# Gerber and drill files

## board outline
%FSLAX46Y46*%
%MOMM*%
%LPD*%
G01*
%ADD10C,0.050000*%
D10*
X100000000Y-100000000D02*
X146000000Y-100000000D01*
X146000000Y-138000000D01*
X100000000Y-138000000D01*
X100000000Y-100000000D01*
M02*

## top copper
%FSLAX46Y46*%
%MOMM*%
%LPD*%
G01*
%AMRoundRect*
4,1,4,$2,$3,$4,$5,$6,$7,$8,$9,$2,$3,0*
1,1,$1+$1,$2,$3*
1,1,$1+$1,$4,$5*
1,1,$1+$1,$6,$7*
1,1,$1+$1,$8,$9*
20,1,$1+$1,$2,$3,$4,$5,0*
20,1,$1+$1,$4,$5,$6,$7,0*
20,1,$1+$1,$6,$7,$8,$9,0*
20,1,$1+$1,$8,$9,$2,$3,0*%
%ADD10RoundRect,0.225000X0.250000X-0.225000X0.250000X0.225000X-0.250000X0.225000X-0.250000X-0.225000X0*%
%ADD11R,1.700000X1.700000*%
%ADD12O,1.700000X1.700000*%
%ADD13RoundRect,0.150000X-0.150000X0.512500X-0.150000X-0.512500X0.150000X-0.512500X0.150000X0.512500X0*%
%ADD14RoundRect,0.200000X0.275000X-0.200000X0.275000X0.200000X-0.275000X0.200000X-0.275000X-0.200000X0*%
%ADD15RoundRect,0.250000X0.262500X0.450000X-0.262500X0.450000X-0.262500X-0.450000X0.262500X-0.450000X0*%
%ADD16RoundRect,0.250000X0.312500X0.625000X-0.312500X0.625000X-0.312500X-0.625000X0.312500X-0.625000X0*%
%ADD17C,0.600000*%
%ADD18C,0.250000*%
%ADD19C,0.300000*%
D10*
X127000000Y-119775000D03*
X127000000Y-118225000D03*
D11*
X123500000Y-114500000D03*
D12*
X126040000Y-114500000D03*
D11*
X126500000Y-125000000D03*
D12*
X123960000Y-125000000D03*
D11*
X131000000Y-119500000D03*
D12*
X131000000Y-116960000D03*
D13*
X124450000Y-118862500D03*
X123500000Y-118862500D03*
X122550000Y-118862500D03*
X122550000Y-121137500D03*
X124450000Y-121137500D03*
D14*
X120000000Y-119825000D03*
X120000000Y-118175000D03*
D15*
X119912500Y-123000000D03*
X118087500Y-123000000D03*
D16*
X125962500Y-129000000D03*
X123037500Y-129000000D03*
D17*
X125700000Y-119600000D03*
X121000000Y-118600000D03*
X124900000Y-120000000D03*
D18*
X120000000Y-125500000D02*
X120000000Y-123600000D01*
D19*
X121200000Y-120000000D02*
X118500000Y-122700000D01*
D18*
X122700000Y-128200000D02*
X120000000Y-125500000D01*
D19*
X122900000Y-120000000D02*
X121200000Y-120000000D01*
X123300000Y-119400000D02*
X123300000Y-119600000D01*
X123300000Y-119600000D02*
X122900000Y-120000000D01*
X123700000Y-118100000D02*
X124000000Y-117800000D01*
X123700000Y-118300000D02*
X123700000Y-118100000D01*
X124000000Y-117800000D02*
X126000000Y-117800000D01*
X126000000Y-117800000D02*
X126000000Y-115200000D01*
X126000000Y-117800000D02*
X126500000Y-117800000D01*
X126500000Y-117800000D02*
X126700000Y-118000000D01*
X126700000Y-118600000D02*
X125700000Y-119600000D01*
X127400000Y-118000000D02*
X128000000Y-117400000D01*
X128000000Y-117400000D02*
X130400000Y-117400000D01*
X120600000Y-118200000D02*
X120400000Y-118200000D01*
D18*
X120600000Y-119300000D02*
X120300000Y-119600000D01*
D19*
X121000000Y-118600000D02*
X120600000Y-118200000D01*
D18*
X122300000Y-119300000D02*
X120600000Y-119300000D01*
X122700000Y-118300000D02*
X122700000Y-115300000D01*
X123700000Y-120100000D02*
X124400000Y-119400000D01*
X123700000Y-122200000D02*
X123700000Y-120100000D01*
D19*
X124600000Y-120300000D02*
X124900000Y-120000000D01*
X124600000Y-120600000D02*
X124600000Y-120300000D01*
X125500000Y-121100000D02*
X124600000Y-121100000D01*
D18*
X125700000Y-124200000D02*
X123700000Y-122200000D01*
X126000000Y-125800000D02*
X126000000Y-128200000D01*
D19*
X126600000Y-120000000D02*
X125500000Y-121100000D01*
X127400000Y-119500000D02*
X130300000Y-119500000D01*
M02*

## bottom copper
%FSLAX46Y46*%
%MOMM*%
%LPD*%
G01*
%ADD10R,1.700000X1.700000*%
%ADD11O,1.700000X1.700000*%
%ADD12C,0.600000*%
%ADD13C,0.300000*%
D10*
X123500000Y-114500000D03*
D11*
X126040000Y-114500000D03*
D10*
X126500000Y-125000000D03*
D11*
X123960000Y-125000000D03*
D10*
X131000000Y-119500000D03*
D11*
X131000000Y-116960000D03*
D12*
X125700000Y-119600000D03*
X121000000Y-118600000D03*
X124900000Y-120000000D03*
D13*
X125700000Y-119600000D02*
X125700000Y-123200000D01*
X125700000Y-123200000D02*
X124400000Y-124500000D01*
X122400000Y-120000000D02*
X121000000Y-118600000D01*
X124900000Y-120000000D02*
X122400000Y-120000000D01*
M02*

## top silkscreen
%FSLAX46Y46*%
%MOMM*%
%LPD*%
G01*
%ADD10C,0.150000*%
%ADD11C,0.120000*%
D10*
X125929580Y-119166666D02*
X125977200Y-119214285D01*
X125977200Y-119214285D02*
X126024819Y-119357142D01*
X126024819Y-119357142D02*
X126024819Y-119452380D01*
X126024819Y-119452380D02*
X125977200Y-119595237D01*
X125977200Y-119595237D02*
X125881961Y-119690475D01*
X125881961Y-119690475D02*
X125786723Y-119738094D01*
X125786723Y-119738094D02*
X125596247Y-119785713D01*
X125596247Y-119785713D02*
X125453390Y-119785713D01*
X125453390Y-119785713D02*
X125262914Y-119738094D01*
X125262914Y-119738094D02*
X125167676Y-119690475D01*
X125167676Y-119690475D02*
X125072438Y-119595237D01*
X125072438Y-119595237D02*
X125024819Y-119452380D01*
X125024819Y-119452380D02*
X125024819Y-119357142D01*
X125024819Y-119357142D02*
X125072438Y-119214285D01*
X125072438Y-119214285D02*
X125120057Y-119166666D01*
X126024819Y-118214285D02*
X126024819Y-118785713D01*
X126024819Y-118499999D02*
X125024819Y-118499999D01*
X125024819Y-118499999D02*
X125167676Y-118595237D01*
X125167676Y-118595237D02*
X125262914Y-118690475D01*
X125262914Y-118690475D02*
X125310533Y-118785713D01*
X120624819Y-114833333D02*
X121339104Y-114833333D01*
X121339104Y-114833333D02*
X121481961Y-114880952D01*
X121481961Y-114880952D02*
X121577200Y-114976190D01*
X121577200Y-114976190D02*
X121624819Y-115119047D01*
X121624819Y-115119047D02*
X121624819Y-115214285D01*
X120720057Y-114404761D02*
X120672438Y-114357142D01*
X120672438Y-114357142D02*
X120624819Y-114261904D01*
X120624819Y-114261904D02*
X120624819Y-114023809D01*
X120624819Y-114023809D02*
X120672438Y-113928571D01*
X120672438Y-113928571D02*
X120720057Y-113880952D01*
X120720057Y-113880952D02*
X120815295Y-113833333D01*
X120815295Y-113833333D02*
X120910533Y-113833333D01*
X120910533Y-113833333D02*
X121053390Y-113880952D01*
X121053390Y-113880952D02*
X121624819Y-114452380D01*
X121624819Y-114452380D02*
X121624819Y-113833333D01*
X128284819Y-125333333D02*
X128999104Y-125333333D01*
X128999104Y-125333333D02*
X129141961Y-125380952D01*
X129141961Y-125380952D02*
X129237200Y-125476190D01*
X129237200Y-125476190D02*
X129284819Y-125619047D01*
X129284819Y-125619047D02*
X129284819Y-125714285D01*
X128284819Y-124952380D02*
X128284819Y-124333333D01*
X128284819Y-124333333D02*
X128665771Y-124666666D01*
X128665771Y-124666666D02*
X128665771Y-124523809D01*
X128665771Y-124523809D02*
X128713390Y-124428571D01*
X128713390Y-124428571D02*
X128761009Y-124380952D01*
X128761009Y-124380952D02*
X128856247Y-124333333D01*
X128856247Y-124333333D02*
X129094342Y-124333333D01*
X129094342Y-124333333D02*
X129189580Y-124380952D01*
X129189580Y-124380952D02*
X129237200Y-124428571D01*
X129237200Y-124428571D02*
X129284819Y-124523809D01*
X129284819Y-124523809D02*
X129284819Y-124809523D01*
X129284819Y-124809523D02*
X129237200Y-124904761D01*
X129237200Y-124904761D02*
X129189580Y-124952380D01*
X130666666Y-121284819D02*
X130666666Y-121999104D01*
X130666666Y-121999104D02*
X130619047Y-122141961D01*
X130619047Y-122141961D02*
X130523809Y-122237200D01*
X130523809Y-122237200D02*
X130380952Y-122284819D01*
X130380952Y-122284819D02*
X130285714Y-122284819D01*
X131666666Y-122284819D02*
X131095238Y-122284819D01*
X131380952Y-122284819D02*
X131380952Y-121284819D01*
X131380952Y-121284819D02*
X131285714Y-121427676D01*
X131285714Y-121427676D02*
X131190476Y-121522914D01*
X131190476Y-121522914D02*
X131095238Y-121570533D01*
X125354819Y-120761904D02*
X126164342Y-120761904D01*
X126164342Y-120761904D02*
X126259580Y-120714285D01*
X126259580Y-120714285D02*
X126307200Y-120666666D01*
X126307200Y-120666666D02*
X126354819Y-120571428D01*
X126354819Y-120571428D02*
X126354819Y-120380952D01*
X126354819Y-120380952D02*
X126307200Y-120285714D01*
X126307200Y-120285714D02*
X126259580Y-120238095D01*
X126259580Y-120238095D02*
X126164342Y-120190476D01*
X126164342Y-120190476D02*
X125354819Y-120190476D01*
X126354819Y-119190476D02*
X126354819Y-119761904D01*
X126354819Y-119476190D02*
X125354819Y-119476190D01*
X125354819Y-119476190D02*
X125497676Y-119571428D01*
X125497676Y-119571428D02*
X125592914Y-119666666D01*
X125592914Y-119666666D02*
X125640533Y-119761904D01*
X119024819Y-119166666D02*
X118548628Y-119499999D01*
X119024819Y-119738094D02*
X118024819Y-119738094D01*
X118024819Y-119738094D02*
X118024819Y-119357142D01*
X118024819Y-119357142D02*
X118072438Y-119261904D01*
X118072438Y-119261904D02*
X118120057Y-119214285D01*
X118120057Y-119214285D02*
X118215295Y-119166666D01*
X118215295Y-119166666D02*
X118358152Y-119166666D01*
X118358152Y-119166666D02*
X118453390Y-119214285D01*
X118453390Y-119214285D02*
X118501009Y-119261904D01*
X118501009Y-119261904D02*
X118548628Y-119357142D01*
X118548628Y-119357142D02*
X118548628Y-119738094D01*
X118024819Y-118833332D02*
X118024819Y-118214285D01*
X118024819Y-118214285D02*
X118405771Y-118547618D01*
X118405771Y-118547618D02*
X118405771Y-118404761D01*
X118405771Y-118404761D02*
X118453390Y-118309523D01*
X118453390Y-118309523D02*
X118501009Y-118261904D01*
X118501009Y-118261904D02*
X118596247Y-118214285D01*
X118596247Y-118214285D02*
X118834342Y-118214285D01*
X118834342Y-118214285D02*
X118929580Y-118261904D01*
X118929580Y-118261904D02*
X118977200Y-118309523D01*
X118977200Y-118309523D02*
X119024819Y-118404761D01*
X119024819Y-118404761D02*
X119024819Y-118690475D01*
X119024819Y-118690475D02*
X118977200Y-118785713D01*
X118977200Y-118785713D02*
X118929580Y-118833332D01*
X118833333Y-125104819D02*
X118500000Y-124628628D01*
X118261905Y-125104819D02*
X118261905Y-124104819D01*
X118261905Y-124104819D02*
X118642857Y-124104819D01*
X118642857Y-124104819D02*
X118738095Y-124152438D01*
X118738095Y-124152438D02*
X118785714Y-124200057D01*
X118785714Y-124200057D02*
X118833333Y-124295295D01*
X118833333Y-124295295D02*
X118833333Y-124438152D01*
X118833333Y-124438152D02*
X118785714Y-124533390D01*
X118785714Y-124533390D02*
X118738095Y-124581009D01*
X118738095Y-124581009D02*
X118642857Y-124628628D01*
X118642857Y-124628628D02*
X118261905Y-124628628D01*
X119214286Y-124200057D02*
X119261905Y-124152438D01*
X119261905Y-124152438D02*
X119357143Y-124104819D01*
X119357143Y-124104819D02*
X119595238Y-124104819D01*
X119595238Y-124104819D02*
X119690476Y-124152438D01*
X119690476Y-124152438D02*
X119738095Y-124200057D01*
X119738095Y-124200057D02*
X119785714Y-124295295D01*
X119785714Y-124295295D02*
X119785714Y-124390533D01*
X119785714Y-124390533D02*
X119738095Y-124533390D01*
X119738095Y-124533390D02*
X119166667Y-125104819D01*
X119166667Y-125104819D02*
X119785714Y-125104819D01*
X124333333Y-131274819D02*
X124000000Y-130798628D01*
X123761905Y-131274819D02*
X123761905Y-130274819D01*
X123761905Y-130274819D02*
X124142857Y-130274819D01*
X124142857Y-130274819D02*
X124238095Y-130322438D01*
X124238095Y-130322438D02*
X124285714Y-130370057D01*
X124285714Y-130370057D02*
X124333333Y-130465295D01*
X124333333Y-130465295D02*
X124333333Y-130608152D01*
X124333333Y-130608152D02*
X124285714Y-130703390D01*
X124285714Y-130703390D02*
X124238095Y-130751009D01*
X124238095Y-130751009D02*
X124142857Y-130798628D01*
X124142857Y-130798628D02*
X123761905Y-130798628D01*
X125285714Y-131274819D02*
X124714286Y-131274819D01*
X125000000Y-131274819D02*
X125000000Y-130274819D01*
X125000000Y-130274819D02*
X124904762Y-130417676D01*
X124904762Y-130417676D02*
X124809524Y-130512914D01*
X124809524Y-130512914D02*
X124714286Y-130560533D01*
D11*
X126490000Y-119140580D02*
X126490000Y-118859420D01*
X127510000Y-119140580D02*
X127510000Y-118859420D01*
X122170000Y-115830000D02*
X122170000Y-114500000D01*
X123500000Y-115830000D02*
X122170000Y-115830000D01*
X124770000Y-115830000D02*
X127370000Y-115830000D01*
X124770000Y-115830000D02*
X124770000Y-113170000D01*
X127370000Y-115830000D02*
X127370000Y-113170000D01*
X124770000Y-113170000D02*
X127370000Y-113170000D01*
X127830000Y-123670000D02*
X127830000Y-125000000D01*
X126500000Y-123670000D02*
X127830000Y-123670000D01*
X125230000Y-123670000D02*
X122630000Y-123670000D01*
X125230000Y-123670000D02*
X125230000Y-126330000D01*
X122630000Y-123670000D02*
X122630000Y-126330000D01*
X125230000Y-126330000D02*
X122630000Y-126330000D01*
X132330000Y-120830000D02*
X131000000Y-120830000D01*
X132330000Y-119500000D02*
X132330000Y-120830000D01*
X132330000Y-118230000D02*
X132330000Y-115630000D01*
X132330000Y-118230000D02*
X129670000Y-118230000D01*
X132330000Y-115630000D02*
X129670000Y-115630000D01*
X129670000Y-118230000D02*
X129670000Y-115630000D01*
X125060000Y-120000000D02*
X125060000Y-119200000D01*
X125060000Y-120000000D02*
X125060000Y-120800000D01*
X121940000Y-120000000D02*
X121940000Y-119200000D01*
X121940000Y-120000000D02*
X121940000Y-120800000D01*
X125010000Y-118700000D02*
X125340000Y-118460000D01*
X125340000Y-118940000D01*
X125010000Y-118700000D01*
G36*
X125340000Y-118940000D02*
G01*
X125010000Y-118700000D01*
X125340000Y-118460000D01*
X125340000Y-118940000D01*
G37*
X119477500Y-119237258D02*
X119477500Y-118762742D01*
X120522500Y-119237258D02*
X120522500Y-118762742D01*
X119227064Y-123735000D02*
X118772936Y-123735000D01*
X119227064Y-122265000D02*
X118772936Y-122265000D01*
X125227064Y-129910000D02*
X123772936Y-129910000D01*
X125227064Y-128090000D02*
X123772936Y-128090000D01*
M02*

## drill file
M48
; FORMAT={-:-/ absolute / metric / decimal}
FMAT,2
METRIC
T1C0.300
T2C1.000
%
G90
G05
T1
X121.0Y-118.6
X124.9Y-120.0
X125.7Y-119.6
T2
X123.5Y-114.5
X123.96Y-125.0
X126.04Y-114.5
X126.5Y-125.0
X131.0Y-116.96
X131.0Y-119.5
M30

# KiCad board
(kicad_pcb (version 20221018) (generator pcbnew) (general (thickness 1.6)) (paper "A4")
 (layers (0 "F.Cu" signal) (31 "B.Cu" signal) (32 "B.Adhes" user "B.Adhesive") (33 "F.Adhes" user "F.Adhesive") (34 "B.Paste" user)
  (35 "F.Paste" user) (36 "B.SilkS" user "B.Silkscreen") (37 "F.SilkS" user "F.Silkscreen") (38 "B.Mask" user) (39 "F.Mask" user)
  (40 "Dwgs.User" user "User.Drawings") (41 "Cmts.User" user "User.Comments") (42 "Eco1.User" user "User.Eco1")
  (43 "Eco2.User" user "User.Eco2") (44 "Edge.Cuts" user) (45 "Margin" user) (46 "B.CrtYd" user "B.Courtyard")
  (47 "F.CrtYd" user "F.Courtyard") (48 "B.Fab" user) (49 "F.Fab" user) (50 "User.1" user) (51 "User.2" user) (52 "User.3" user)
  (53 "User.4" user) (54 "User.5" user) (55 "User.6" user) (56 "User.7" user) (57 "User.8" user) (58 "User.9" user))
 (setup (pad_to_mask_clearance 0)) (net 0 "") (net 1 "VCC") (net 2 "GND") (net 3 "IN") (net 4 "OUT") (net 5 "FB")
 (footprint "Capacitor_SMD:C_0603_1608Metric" (layer "F.Cu") (at 127 119 90)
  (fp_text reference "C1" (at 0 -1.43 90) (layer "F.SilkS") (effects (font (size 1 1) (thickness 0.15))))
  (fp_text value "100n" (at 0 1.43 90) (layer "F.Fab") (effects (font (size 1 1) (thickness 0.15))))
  (fp_line (start -0.14058 -0.51) (end 0.14058 -0.51) (stroke (width 0.12) (type solid)) (layer "F.SilkS"))
  (fp_line (start -0.14058 0.51) (end 0.14058 0.51) (stroke (width 0.12) (type solid)) (layer "F.SilkS"))
  (pad "1" smd roundrect (at -0.775 0 90) (size 0.9 0.95) (layers "F.Cu" "F.Paste" "F.Mask") (roundrect_rratio 0.25) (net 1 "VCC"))
  (pad "2" smd roundrect (at 0.775 0 90) (size 0.9 0.95) (layers "F.Cu" "F.Paste" "F.Mask") (roundrect_rratio 0.25) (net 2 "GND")))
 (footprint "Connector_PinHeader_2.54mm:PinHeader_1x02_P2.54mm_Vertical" (layer "F.Cu") (at 123.5 114.5 90)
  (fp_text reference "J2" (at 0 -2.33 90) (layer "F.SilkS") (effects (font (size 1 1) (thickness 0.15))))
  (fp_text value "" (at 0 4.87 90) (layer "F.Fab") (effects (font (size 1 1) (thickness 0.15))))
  (fp_line (start -1.33 -1.33) (end 0 -1.33) (stroke (width 0.12) (type solid)) (layer "F.SilkS"))
  (fp_line (start -1.33 0) (end -1.33 -1.33) (stroke (width 0.12) (type solid)) (layer "F.SilkS"))
  (fp_line (start -1.33 1.27) (end -1.33 3.87) (stroke (width 0.12) (type solid)) (layer "F.SilkS"))
  (fp_line (start -1.33 1.27) (end 1.33 1.27) (stroke (width 0.12) (type solid)) (layer "F.SilkS"))
  (fp_line (start -1.33 3.87) (end 1.33 3.87) (stroke (width 0.12) (type solid)) (layer "F.SilkS"))
  (fp_line (start 1.33 1.27) (end 1.33 3.87) (stroke (width 0.12) (type solid)) (layer "F.SilkS"))
  (pad "1" thru_hole rect (at 0 0 90) (size 1.7 1.7) (drill 1) (layers "*.Cu" "*.Mask") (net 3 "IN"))
  (pad "2" thru_hole oval (at 0 2.54 90) (size 1.7 1.7) (drill 1) (layers "*.Cu" "*.Mask") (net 2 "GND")))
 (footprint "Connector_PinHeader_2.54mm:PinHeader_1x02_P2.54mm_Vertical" (layer "F.Cu") (at 126.5 125 -90)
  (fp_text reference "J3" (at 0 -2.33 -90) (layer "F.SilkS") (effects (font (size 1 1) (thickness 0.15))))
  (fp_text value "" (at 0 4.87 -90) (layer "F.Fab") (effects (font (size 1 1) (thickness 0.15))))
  (fp_line (start -1.33 -1.33) (end 0 -1.33) (stroke (width 0.12) (type solid)) (layer "F.SilkS"))
  (fp_line (start -1.33 0) (end -1.33 -1.33) (stroke (width 0.12) (type solid)) (layer "F.SilkS"))
  (fp_line (start -1.33 1.27) (end -1.33 3.87) (stroke (width 0.12) (type solid)) (layer "F.SilkS"))
  (fp_line (start -1.33 1.27) (end 1.33 1.27) (stroke (width 0.12) (type solid)) (layer "F.SilkS"))
  (fp_line (start -1.33 3.87) (end 1.33 3.87) (stroke (width 0.12) (type solid)) (layer "F.SilkS"))
  (fp_line (start 1.33 1.27) (end 1.33 3.87) (stroke (width 0.12) (type solid)) (layer "F.SilkS"))
  (pad "1" thru_hole rect (at 0 0 270) (size 1.7 1.7) (drill 1) (layers "*.Cu" "*.Mask") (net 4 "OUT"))
  (pad "2" thru_hole oval (at 0 2.54 270) (size 1.7 1.7) (drill 1) (layers "*.Cu" "*.Mask") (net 2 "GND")))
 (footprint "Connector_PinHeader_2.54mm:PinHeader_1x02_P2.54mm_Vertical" (layer "F.Cu") (at 131 119.5 180)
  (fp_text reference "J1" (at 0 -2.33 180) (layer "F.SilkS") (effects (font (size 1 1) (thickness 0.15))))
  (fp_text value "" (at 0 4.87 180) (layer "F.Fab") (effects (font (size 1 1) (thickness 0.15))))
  (fp_line (start -1.33 -1.33) (end 0 -1.33) (stroke (width 0.12) (type solid)) (layer "F.SilkS"))
  (fp_line (start -1.33 0) (end -1.33 -1.33) (stroke (width 0.12) (type solid)) (layer "F.SilkS"))
  (fp_line (start -1.33 1.27) (end -1.33 3.87) (stroke (width 0.12) (type solid)) (layer "F.SilkS"))
  (fp_line (start -1.33 1.27) (end 1.33 1.27) (stroke (width 0.12) (type solid)) (layer "F.SilkS"))
  (fp_line (start -1.33 3.87) (end 1.33 3.87) (stroke (width 0.12) (type solid)) (layer "F.SilkS"))
  (fp_line (start 1.33 1.27) (end 1.33 3.87) (stroke (width 0.12) (type solid)) (layer "F.SilkS"))
  (pad "1" thru_hole rect (at 0 0 180) (size 1.7 1.7) (drill 1) (layers "*.Cu" "*.Mask") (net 1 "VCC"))
  (pad "2" thru_hole oval (at 0 2.54 180) (size 1.7 1.7) (drill 1) (layers "*.Cu" "*.Mask") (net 2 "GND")))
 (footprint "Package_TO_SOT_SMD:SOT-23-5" (layer "F.Cu") (at 123.5 120 -90)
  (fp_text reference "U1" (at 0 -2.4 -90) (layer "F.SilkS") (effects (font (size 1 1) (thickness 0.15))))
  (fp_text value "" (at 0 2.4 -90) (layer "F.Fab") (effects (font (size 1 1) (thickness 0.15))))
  (fp_line (start 0 -1.56) (end -0.8 -1.56) (stroke (width 0.12) (type solid)) (layer "F.SilkS"))
  (fp_line (start 0 -1.56) (end 0.8 -1.56) (stroke (width 0.12) (type solid)) (layer "F.SilkS"))
  (fp_line (start 0 1.56) (end -0.8 1.56) (stroke (width 0.12) (type solid)) (layer "F.SilkS"))
  (fp_line (start 0 1.56) (end 0.8 1.56) (stroke (width 0.12) (type solid)) (layer "F.SilkS"))
  (fp_poly
   (pts (xy -1.3 -1.51) (xy -1.54 -1.84) (xy -1.06 -1.84) (xy -1.3 -1.51)) (stroke (width 0.12) (type solid)) (fill solid) (layer "F.SilkS"))
  (pad "1" smd roundrect (at -1.1375 -0.95 270) (size 1.325 0.6) (layers "F.Cu" "F.Paste" "F.Mask") (roundrect_rratio 0.25) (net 4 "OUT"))
  (pad "2" smd roundrect (at -1.1375 0 270) (size 1.325 0.6) (layers "F.Cu" "F.Paste" "F.Mask") (roundrect_rratio 0.25) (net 2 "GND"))
  (pad "3" smd roundrect (at -1.1375 0.95 270) (size 1.325 0.6) (layers "F.Cu" "F.Paste" "F.Mask") (roundrect_rratio 0.25) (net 3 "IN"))
  (pad "4" smd roundrect (at 1.1375 0.95 270) (size 1.325 0.6) (layers "F.Cu" "F.Paste" "F.Mask") (roundrect_rratio 0.25))
  (pad "5" smd roundrect (at 1.1375 -0.95 270) (size 1.325 0.6) (layers "F.Cu" "F.Paste" "F.Mask") (roundrect_rratio 0.25) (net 1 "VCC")))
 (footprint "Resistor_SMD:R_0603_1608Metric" (layer "F.Cu") (at 120 119 90)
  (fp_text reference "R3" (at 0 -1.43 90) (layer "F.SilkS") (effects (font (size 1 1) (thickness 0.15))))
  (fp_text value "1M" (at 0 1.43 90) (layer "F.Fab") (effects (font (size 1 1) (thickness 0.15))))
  (fp_line (start -0.237258 -0.5225) (end 0.237258 -0.5225) (stroke (width 0.12) (type solid)) (layer "F.SilkS"))
  (fp_line (start -0.237258 0.5225) (end 0.237258 0.5225) (stroke (width 0.12) (type solid)) (layer "F.SilkS"))
  (pad "1" smd roundrect (at -0.825 0 90) (size 0.8 0.95) (layers "F.Cu" "F.Paste" "F.Mask") (roundrect_rratio 0.25) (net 3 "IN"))
  (pad "2" smd roundrect (at 0.825 0 90) (size 0.8 0.95) (layers "F.Cu" "F.Paste" "F.Mask") (roundrect_rratio 0.25) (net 1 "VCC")))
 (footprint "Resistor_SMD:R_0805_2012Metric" (layer "F.Cu") (at 119 123 180)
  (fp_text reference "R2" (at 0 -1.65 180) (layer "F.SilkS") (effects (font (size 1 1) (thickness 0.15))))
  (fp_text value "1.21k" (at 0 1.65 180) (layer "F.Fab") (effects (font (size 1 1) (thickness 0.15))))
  (fp_line (start -0.227064 -0.735) (end 0.227064 -0.735) (stroke (width 0.12) (type solid)) (layer "F.SilkS"))
  (fp_line (start -0.227064 0.735) (end 0.227064 0.735) (stroke (width 0.12) (type solid)) (layer "F.SilkS"))
  (pad "1" smd roundrect (at -0.9125 0 180) (size 1.025 1.4) (layers "F.Cu" "F.Paste" "F.Mask") (roundrect_rratio 0.243902) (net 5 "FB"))
  (pad "2" smd roundrect (at 0.9125 0 180) (size 1.025 1.4) (layers "F.Cu" "F.Paste" "F.Mask") (roundrect_rratio 0.243902) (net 2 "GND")))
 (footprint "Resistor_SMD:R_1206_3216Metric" (layer "F.Cu") (at 124.5 129 180)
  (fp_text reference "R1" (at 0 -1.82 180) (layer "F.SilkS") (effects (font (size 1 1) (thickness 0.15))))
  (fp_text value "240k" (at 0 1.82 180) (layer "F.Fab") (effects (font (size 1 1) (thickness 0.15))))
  (fp_line (start -0.727064 -0.91) (end 0.727064 -0.91) (stroke (width 0.12) (type solid)) (layer "F.SilkS"))
  (fp_line (start -0.727064 0.91) (end 0.727064 0.91) (stroke (width 0.12) (type solid)) (layer "F.SilkS"))
  (pad "1" smd roundrect (at -1.4625 0 180) (size 1.125 1.75) (layers "F.Cu" "F.Paste" "F.Mask") (roundrect_rratio 0.222222) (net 4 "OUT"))
  (pad "2" smd roundrect (at 1.4625 0 180) (size 1.125 1.75) (layers "F.Cu" "F.Paste" "F.Mask") (roundrect_rratio 0.222222) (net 5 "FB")))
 (gr_rect (start 100 100) (end 146 138) (stroke (width 0.05) (type default)) (fill none) (layer "Edge.Cuts"))
 (segment (start 120 125.5) (end 120 123.6) (width 0.25) (layer "F.Cu") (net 5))
 (segment (start 121.2 120) (end 118.5 122.7) (width 0.3) (layer "F.Cu") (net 2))
 (segment (start 122.7 128.2) (end 120 125.5) (width 0.25) (layer "F.Cu") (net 5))
 (segment (start 122.9 120) (end 121.2 120) (width 0.3) (layer "F.Cu") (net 2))
 (segment (start 123.3 119.4) (end 123.3 119.6) (width 0.3) (layer "F.Cu") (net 2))
 (segment (start 123.3 119.6) (end 122.9 120) (width 0.3) (layer "F.Cu") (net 2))
 (segment (start 123.7 118.1) (end 124 117.8) (width 0.3) (layer "F.Cu") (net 2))
 (segment (start 123.7 118.3) (end 123.7 118.1) (width 0.3) (layer "F.Cu") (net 2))
 (segment (start 124 117.8) (end 126 117.8) (width 0.3) (layer "F.Cu") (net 2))
 (segment (start 126 117.8) (end 126 115.2) (width 0.3) (layer "F.Cu") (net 2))
 (segment (start 126 117.8) (end 126.5 117.8) (width 0.3) (layer "F.Cu") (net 2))
 (segment (start 126.5 117.8) (end 126.7 118) (width 0.3) (layer "F.Cu") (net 2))
 (segment (start 126.7 118.6) (end 125.7 119.6) (width 0.3) (layer "F.Cu") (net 2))
 (segment (start 127.4 118) (end 128 117.4) (width 0.3) (layer "F.Cu") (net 2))
 (segment (start 128 117.4) (end 130.4 117.4) (width 0.3) (layer "F.Cu") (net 2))
 (via (at 125.7 119.6) (size 0.6) (drill 0.3) (layers "F.Cu" "B.Cu") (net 2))
 (segment (start 120.6 118.2) (end 120.4 118.2) (width 0.3) (layer "F.Cu") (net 1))
 (segment (start 120.6 119.3) (end 120.3 119.6) (width 0.25) (layer "F.Cu") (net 3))
 (segment (start 121 118.6) (end 120.6 118.2) (width 0.3) (layer "F.Cu") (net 1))
 (segment (start 122.3 119.3) (end 120.6 119.3) (width 0.25) (layer "F.Cu") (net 3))
 (segment (start 122.7 118.3) (end 122.7 115.3) (width 0.25) (layer "F.Cu") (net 3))
 (segment (start 123.7 120.1) (end 124.4 119.4) (width 0.25) (layer "F.Cu") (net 4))
 (segment (start 123.7 122.2) (end 123.7 120.1) (width 0.25) (layer "F.Cu") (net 4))
 (segment (start 124.6 120.3) (end 124.9 120) (width 0.3) (layer "F.Cu") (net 1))
 (segment (start 124.6 120.6) (end 124.6 120.3) (width 0.3) (layer "F.Cu") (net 1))
 (segment (start 125.5 121.1) (end 124.6 121.1) (width 0.3) (layer "F.Cu") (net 1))
 (segment (start 125.7 119.6) (end 125.7 123.2) (width 0.3) (layer "B.Cu") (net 2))
 (segment (start 125.7 123.2) (end 124.4 124.5) (width 0.3) (layer "B.Cu") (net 2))
 (segment (start 125.7 124.2) (end 123.7 122.2) (width 0.25) (layer "F.Cu") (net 4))
 (segment (start 126 125.8) (end 126 128.2) (width 0.25) (layer "F.Cu") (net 4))
 (segment (start 126.6 120) (end 125.5 121.1) (width 0.3) (layer "F.Cu") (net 1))
 (segment (start 127.4 119.5) (end 130.3 119.5) (width 0.3) (layer "F.Cu") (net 1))
 (via (at 121 118.6) (size 0.6) (drill 0.3) (layers "F.Cu" "B.Cu") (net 1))
 (via (at 124.9 120) (size 0.6) (drill 0.3) (layers "F.Cu" "B.Cu") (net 1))
 (segment (start 122.4 120) (end 121 118.6) (width 0.3) (layer "B.Cu") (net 1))
 (segment (start 124.9 120) (end 122.4 120) (width 0.3) (layer "B.Cu") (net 1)))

